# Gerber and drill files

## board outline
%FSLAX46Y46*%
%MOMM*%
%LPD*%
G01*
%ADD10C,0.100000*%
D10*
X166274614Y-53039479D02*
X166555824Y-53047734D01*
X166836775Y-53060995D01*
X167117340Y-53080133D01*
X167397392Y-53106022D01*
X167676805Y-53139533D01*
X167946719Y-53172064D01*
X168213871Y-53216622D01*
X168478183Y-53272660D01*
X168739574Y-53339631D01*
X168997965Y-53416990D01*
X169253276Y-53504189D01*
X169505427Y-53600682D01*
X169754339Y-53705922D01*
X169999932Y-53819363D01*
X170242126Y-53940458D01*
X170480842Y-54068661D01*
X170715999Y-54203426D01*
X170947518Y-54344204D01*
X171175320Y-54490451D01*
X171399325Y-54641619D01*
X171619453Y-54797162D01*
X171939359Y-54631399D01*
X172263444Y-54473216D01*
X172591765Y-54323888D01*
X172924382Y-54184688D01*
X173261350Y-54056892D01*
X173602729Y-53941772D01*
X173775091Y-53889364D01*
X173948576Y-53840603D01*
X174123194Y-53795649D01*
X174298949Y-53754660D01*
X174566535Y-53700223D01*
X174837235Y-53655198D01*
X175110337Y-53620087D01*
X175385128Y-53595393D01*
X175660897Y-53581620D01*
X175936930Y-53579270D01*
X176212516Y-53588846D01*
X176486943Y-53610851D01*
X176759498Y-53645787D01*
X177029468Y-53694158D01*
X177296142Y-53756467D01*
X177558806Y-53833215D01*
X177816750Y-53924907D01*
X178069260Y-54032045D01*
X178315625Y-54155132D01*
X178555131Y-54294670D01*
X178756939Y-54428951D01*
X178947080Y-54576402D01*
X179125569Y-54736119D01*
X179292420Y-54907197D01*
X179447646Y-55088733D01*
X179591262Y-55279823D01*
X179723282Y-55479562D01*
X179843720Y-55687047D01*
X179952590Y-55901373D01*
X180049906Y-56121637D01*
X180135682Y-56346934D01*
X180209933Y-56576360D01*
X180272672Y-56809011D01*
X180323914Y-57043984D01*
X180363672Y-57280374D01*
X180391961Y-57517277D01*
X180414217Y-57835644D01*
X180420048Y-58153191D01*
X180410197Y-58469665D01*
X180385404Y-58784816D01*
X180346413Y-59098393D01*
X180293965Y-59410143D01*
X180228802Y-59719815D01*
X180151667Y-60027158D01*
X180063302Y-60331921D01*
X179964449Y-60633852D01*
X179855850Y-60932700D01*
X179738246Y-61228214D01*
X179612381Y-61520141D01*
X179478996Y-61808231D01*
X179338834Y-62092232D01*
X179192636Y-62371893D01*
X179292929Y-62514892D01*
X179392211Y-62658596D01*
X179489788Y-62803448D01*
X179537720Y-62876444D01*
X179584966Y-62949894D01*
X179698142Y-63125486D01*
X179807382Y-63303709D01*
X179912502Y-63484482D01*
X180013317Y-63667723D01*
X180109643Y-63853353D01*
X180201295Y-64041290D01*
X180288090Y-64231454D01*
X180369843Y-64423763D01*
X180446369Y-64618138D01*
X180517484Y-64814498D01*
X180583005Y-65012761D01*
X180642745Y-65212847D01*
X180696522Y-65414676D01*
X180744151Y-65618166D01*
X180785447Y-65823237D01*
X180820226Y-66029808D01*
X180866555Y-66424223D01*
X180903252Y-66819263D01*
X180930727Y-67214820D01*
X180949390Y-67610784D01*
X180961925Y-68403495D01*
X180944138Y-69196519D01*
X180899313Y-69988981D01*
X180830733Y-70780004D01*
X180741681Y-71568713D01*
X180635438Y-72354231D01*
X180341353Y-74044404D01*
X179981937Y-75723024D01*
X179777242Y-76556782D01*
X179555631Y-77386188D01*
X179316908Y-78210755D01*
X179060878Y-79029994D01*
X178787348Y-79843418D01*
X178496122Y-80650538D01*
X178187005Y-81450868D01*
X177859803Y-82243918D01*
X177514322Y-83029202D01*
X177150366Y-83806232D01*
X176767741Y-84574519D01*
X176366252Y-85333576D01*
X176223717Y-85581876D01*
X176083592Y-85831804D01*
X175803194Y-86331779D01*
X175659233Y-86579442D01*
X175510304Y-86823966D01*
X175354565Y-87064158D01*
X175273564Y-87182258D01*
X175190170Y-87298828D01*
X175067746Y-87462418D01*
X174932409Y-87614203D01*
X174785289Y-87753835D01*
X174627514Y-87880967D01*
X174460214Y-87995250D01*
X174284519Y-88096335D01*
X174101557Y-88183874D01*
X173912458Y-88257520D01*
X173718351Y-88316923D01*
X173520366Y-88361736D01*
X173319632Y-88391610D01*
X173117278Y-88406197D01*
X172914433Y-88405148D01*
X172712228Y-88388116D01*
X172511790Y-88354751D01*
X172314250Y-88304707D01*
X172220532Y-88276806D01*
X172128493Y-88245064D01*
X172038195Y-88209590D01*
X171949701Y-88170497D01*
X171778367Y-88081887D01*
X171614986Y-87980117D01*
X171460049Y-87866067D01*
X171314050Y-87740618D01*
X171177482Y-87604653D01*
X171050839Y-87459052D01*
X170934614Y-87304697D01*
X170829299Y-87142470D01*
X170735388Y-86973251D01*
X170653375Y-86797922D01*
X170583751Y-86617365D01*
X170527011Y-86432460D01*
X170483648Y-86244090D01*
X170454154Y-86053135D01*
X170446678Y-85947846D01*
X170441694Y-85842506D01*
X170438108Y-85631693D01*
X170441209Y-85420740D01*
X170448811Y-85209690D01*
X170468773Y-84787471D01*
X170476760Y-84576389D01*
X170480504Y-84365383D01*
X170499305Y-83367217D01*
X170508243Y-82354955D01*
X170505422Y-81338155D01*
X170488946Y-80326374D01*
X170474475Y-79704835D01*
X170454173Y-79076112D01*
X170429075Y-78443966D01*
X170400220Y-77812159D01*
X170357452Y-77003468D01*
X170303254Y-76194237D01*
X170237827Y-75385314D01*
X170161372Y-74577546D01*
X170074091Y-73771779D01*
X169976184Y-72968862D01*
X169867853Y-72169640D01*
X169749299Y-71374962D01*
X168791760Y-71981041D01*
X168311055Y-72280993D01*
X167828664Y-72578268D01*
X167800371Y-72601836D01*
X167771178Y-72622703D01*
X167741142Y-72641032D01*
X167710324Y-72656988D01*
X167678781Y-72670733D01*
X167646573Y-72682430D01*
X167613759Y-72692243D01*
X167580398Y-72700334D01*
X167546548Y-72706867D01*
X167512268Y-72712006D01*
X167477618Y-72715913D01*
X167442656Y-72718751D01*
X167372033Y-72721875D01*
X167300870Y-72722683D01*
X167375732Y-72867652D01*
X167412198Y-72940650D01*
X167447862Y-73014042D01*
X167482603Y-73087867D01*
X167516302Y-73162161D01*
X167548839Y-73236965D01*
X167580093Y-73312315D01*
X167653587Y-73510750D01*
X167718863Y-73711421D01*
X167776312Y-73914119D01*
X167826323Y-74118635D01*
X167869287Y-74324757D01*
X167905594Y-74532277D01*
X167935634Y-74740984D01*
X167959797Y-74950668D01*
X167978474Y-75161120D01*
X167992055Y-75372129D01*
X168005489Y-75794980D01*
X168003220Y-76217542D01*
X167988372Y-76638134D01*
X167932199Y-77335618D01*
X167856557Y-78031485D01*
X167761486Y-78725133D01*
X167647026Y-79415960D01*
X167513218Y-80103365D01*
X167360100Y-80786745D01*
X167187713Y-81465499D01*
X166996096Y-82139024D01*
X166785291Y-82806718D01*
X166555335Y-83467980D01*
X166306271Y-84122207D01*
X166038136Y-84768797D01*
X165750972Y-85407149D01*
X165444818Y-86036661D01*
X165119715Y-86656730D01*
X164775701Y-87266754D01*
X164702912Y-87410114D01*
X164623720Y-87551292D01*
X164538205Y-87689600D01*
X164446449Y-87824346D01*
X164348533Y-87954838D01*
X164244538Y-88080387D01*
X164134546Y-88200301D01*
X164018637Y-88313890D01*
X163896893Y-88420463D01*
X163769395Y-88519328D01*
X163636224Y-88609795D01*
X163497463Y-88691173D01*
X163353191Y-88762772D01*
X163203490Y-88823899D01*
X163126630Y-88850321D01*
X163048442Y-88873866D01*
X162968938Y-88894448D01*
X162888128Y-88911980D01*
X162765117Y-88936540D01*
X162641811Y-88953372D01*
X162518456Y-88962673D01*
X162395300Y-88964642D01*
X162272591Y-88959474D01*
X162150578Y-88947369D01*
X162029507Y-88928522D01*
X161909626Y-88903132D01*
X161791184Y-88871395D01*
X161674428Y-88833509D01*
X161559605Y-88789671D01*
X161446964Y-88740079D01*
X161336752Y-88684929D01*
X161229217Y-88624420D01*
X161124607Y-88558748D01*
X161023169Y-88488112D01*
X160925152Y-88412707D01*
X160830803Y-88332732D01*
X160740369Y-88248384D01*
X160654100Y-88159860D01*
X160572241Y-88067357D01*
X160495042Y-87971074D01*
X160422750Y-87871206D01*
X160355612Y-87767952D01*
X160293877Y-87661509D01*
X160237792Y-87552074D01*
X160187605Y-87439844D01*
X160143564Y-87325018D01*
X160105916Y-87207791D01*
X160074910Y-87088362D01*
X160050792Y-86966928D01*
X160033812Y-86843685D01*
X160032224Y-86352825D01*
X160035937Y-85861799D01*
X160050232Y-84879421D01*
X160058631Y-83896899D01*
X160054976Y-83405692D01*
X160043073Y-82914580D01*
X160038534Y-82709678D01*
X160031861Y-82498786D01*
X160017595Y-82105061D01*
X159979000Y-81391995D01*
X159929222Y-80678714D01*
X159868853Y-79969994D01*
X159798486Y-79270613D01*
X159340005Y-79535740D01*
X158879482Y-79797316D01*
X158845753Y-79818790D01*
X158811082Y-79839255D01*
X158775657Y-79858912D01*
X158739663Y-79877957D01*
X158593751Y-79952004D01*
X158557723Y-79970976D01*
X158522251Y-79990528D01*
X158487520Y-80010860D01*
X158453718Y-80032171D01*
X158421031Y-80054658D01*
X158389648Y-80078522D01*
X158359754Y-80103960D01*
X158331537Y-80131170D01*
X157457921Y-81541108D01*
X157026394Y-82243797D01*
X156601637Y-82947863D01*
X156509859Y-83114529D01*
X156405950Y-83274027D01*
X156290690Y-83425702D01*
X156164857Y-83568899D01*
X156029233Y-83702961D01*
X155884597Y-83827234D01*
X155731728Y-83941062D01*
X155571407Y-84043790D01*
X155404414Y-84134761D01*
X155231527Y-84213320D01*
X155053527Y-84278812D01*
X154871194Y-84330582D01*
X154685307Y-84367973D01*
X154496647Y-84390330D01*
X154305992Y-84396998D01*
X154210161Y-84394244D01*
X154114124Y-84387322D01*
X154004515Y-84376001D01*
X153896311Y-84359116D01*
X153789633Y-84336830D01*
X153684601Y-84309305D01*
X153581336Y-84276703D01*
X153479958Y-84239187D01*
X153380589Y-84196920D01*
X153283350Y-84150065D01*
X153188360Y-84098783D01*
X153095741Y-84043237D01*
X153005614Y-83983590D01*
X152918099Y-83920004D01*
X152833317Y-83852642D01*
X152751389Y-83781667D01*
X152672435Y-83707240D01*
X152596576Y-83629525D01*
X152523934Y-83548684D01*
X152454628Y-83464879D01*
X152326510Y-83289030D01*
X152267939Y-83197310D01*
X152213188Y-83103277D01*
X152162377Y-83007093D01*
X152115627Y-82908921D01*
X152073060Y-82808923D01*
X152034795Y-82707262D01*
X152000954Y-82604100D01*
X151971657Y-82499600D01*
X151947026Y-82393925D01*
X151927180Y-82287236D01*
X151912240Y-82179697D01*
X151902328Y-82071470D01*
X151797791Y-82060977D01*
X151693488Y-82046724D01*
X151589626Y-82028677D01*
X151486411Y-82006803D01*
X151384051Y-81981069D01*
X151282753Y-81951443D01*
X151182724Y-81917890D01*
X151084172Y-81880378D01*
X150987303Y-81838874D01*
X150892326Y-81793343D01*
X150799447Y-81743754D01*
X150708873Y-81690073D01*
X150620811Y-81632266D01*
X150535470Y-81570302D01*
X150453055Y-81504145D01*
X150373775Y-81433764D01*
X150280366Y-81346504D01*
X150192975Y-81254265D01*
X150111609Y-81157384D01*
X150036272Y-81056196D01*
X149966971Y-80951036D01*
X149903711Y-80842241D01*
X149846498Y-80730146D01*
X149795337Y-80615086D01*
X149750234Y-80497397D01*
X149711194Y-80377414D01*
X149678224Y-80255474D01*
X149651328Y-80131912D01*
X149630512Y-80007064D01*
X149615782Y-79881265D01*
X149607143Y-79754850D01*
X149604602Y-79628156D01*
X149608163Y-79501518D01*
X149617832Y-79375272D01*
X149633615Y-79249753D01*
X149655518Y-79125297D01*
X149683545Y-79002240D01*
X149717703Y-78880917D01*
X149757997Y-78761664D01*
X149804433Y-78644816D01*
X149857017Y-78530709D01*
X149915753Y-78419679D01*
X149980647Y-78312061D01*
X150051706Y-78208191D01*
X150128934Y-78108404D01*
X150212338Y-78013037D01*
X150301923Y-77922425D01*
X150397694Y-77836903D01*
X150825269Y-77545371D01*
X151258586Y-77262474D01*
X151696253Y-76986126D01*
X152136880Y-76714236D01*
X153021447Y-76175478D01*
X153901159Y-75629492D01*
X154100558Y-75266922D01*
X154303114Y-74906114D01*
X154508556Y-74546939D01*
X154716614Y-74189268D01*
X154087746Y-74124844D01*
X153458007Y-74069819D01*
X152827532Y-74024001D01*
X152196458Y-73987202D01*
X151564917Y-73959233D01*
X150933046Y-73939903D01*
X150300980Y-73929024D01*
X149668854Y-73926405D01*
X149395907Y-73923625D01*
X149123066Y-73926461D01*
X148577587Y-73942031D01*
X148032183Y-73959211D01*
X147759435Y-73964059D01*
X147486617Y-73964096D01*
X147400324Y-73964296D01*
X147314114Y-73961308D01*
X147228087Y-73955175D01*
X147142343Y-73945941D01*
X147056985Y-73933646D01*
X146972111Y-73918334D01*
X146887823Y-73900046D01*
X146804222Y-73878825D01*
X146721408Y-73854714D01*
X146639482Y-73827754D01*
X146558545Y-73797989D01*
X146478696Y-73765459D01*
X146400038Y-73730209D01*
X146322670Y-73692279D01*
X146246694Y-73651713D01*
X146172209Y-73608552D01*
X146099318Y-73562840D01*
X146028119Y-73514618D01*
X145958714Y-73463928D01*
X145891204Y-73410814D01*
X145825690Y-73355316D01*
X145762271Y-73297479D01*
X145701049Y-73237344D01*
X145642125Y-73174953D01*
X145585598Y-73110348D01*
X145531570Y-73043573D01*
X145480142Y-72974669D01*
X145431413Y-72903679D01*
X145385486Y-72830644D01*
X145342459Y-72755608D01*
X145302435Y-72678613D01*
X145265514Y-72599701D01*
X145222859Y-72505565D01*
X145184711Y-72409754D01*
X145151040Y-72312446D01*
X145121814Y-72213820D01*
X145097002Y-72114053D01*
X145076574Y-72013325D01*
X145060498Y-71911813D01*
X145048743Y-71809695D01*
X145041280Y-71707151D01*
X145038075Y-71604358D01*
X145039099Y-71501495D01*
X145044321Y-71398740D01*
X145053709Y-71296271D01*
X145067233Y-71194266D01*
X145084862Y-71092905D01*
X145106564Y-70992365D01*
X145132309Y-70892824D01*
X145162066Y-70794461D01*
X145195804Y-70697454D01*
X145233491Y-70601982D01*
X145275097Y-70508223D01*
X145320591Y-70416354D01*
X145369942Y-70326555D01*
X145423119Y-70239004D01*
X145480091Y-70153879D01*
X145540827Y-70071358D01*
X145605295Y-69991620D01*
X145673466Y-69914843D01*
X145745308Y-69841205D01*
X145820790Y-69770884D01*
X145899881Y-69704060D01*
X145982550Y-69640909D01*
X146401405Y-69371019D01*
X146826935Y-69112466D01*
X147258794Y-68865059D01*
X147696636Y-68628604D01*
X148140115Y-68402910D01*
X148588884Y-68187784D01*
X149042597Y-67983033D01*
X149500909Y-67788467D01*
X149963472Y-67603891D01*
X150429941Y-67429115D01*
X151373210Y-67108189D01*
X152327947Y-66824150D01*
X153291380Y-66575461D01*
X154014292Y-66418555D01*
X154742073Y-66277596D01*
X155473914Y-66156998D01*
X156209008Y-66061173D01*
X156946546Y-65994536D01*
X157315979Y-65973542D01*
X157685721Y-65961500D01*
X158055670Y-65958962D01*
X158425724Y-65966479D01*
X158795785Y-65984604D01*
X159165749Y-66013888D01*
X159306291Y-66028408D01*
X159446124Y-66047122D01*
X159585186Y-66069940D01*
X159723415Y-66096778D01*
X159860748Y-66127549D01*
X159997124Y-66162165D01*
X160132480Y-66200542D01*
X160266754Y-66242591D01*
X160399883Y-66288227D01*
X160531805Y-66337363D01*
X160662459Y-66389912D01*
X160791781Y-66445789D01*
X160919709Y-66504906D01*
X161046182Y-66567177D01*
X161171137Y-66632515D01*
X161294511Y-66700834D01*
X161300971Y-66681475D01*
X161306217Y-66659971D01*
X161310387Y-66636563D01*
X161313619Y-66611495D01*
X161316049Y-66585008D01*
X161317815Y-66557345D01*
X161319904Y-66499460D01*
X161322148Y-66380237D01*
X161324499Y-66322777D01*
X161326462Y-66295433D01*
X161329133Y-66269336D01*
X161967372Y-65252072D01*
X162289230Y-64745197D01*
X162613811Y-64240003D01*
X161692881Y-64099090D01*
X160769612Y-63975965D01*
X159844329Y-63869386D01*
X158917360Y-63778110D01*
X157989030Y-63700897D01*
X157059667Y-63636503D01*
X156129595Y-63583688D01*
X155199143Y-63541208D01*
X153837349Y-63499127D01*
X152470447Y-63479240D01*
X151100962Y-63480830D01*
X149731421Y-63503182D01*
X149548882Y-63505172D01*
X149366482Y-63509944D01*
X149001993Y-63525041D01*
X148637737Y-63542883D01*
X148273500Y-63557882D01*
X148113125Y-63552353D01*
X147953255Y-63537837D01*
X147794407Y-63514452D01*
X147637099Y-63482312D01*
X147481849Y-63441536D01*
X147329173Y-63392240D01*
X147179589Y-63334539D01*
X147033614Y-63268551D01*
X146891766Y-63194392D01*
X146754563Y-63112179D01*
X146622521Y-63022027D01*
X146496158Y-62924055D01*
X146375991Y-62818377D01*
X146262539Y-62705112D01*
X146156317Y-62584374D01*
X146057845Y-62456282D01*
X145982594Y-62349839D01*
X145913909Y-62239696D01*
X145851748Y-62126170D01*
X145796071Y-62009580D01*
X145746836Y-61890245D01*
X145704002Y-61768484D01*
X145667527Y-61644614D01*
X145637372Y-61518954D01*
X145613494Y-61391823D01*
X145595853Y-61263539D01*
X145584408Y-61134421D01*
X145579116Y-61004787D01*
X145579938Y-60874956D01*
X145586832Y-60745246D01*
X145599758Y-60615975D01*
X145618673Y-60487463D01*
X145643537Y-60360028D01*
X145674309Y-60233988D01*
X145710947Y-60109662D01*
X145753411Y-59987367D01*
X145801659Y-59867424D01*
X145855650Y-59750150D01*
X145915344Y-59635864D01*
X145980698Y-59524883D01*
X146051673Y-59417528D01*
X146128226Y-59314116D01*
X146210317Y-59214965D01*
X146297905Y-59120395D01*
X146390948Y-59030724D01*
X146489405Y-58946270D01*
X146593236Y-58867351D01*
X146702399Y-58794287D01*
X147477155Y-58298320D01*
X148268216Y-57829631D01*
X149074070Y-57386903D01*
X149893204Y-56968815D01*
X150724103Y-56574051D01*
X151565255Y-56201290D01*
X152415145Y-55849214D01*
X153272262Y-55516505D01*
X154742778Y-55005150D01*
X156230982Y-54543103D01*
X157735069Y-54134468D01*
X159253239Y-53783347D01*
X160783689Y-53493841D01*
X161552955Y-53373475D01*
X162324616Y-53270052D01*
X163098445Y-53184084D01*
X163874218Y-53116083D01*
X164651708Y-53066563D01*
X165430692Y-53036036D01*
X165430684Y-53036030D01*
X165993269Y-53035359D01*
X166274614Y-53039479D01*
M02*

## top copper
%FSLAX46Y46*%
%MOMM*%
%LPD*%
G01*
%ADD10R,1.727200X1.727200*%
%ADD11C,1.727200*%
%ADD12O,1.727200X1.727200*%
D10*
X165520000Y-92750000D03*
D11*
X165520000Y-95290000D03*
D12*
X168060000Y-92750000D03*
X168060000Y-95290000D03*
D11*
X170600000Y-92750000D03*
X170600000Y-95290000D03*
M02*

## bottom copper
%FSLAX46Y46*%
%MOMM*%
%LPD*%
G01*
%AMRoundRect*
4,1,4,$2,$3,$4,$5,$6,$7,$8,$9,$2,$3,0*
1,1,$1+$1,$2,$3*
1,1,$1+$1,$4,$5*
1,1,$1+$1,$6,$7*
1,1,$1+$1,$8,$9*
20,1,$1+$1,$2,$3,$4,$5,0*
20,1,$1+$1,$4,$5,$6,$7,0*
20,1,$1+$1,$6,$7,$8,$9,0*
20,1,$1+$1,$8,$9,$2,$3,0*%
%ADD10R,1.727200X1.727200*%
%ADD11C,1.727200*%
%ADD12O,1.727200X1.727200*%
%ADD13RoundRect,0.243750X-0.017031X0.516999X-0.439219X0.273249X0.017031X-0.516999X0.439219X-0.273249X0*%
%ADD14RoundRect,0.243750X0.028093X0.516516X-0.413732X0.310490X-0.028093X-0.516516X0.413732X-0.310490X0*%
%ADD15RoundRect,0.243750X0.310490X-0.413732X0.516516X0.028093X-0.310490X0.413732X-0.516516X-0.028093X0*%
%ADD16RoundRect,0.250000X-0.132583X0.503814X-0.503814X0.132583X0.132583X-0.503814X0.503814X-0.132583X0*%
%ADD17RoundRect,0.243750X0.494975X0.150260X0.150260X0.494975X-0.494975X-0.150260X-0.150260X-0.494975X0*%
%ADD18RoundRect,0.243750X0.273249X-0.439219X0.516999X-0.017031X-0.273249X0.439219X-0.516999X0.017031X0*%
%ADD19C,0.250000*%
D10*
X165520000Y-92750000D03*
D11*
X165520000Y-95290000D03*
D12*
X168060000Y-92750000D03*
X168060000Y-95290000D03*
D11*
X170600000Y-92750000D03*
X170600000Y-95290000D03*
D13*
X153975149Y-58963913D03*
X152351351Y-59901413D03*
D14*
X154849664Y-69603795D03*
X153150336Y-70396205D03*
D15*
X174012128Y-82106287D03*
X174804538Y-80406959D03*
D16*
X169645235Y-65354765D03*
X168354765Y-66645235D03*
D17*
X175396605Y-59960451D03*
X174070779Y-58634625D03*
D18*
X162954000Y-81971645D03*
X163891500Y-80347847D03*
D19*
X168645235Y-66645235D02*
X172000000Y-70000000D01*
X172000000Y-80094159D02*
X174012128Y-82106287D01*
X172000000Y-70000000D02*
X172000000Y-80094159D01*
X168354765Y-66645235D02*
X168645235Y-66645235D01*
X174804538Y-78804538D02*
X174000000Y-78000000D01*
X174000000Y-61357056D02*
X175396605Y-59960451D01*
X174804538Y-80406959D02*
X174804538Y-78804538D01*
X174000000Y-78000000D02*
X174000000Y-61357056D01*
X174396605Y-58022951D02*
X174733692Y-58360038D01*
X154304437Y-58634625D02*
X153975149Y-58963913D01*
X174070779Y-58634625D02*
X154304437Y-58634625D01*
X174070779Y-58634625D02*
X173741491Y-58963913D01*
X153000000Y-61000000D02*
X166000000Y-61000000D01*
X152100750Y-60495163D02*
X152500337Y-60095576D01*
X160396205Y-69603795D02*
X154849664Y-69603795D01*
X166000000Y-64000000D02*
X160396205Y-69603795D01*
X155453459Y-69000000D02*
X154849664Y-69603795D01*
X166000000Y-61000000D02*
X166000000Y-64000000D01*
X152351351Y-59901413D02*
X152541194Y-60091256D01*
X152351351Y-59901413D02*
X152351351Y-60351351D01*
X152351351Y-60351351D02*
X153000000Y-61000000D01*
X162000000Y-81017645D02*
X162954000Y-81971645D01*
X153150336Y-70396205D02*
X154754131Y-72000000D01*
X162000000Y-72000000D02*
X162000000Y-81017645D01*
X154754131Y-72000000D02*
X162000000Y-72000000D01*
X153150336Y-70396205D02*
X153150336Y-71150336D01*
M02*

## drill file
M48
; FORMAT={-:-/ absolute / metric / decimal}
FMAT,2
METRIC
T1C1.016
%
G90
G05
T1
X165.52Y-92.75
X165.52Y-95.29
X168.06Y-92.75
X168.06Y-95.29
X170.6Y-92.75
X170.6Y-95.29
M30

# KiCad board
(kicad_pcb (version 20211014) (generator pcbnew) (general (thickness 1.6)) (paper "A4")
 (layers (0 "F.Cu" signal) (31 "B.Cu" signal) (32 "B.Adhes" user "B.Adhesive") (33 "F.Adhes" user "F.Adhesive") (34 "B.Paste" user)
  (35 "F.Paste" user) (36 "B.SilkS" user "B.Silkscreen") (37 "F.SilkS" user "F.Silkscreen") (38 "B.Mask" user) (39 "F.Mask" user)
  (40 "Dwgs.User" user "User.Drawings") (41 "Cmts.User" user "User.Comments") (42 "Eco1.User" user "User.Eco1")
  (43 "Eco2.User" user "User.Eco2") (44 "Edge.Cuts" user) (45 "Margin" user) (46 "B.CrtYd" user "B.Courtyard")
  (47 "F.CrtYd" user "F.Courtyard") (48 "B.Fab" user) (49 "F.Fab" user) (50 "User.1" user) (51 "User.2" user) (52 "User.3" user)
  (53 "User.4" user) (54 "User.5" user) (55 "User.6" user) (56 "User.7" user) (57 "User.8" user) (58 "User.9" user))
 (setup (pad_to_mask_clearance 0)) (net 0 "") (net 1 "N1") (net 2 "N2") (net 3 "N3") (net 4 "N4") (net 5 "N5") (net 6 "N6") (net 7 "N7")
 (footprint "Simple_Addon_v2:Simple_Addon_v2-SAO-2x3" (layer "F.Cu") (at 168 94)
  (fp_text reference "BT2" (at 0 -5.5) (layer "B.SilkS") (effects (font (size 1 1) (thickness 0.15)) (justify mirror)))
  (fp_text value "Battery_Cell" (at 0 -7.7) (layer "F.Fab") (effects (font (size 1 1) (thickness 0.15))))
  (pad "1" thru_hole rect locked (at -2.48 -1.25 270) (size 1.7272 1.7272) (drill 1.016) (layers *.Cu *.Mask) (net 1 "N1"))
  (pad "2" thru_hole circle locked (at -2.48 1.29 270) (size 1.7272 1.7272) (drill 1.016) (layers *.Cu *.Mask) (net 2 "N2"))
  (pad "3" thru_hole oval locked (at 0.06 -1.25 270) (size 1.7272 1.7272) (drill 1.016) (layers *.Cu *.Mask))
  (pad "4" thru_hole oval locked (at 0.06 1.29 270) (size 1.7272 1.7272) (drill 1.016) (layers *.Cu *.Mask))
  (pad "5" thru_hole circle locked (at 2.6 -1.25 270) (size 1.7272 1.7272) (drill 1.016) (layers *.Cu *.Mask))
  (pad "6" thru_hole circle locked (at 2.6 1.29 270) (size 1.7272 1.7272) (drill 1.016) (layers *.Cu *.Mask)))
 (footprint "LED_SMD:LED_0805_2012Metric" (layer "B.Cu") (at 153.16325 59.432663 -150)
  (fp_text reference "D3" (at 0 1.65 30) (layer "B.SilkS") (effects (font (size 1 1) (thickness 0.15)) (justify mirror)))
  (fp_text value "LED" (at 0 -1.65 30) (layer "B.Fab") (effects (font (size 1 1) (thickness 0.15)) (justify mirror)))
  (pad "1" smd roundrect (at -0.9375 0 210) (size 0.975 1.4) (layers "B.Cu" "B.Paste" "B.Mask") (roundrect_rratio 0.25) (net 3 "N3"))
  (pad "2" smd roundrect (at 0.9375 0 210) (size 0.975 1.4) (layers "B.Cu" "B.Paste" "B.Mask") (roundrect_rratio 0.25) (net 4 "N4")))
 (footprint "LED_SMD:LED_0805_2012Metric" (layer "B.Cu") (at 154 70 -155)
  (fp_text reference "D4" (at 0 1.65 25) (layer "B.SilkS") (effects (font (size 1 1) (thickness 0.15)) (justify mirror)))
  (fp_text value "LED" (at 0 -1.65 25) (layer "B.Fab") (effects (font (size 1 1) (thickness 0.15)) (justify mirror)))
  (pad "1" smd roundrect (at -0.9375 0 205) (size 0.975 1.4) (layers "B.Cu" "B.Paste" "B.Mask") (roundrect_rratio 0.25) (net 4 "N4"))
  (pad "2" smd roundrect (at 0.9375 0 205) (size 0.975 1.4) (layers "B.Cu" "B.Paste" "B.Mask") (roundrect_rratio 0.25) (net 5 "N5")))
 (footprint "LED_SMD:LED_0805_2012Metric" (layer "B.Cu") (at 174.408333 81.256623 65)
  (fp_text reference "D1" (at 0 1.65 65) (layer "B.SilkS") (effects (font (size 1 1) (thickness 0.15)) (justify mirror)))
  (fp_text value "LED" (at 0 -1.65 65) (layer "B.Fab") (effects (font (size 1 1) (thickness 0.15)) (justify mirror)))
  (pad "1" smd roundrect (at -0.9375 0 65) (size 0.975 1.4) (layers "B.Cu" "B.Paste" "B.Mask") (roundrect_rratio 0.25) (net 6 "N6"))
  (pad "2" smd roundrect (at 0.9375 0 65) (size 0.975 1.4) (layers "B.Cu" "B.Paste" "B.Mask") (roundrect_rratio 0.25) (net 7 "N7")))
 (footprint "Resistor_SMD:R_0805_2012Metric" (layer "B.Cu") (at 169 66 -135)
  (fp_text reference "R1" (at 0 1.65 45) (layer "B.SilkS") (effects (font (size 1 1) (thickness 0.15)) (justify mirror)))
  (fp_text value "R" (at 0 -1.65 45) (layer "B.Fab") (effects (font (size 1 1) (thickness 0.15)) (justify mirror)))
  (pad "1" smd roundrect (at -0.9125 0 225) (size 1.025 1.4) (layers "B.Cu" "B.Paste" "B.Mask") (roundrect_rratio 0.243902) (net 2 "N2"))
  (pad "2" smd roundrect (at 0.9125 0 225) (size 1.025 1.4) (layers "B.Cu" "B.Paste" "B.Mask") (roundrect_rratio 0.243902) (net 6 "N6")))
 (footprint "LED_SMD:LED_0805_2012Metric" (layer "B.Cu") (at 174.733692 59.297538 135)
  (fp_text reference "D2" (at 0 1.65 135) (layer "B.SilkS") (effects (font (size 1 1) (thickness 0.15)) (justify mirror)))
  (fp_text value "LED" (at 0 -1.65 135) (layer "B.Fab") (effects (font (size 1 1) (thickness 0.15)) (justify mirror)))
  (pad "1" smd roundrect (at -0.9375 0 135) (size 0.975 1.4) (layers "B.Cu" "B.Paste" "B.Mask") (roundrect_rratio 0.25) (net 7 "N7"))
  (pad "2" smd roundrect (at 0.9375 0 135) (size 0.975 1.4) (layers "B.Cu" "B.Paste" "B.Mask") (roundrect_rratio 0.25) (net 3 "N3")))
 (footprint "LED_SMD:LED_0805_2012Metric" (layer "B.Cu") (at 163.42275 81.159746 60)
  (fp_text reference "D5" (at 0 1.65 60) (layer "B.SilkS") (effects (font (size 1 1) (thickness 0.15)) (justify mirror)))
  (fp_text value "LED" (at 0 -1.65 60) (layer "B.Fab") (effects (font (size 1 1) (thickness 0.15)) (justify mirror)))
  (pad "1" smd roundrect (at -0.9375 0 60) (size 0.975 1.4) (layers "B.Cu" "B.Paste" "B.Mask") (roundrect_rratio 0.25) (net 5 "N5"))
  (pad "2" smd roundrect (at 0.9375 0 60) (size 0.975 1.4) (layers "B.Cu" "B.Paste" "B.Mask") (roundrect_rratio 0.25) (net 1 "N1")))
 (gr_poly
  (pts (xy 166.274614 53.039479) (xy 166.555824 53.047734) (xy 166.836775 53.060995) (xy 167.11734 53.080133) (xy 167.397392 53.106022)
   (xy 167.676805 53.139533) (xy 167.946719 53.172064) (xy 168.213871 53.216622) (xy 168.478183 53.27266) (xy 168.739574 53.339631)
   (xy 168.997965 53.41699) (xy 169.253276 53.504189) (xy 169.505427 53.600682) (xy 169.754339 53.705922) (xy 169.999932 53.819363)
   (xy 170.242126 53.940458) (xy 170.480842 54.068661) (xy 170.715999 54.203426) (xy 170.947518 54.344204) (xy 171.17532 54.490451)
   (xy 171.399325 54.641619) (xy 171.619453 54.797162) (xy 171.939359 54.631399) (xy 172.263444 54.473216) (xy 172.591765 54.323888)
   (xy 172.924382 54.184688) (xy 173.26135 54.056892) (xy 173.602729 53.941772) (xy 173.775091 53.889364) (xy 173.948576 53.840603)
   (xy 174.123194 53.795649) (xy 174.298949 53.75466) (xy 174.566535 53.700223) (xy 174.837235 53.655198) (xy 175.110337 53.620087)
   (xy 175.385128 53.595393) (xy 175.660897 53.58162) (xy 175.93693 53.57927) (xy 176.212516 53.588846) (xy 176.486943 53.610851)
   (xy 176.759498 53.645787) (xy 177.029468 53.694158) (xy 177.296142 53.756467) (xy 177.558806 53.833215) (xy 177.81675 53.924907)
   (xy 178.06926 54.032045) (xy 178.315625 54.155132) (xy 178.555131 54.29467) (xy 178.756939 54.428951) (xy 178.94708 54.576402)
   (xy 179.125569 54.736119) (xy 179.29242 54.907197) (xy 179.447646 55.088733) (xy 179.591262 55.279823) (xy 179.723282 55.479562)
   (xy 179.84372 55.687047) (xy 179.95259 55.901373) (xy 180.049906 56.121637) (xy 180.135682 56.346934) (xy 180.209933 56.57636)
   (xy 180.272672 56.809011) (xy 180.323914 57.043984) (xy 180.363672 57.280374) (xy 180.391961 57.517277) (xy 180.414217 57.835644)
   (xy 180.420048 58.153191) (xy 180.410197 58.469665) (xy 180.385404 58.784816) (xy 180.346413 59.098393) (xy 180.293965 59.410143)
   (xy 180.228802 59.719815) (xy 180.151667 60.027158) (xy 180.063302 60.331921) (xy 179.964449 60.633852) (xy 179.85585 60.9327)
   (xy 179.738246 61.228214) (xy 179.612381 61.520141) (xy 179.478996 61.808231) (xy 179.338834 62.092232) (xy 179.192636 62.371893)
   (xy 179.292929 62.514892) (xy 179.392211 62.658596) (xy 179.489788 62.803448) (xy 179.53772 62.876444) (xy 179.584966 62.949894)
   (xy 179.698142 63.125486) (xy 179.807382 63.303709) (xy 179.912502 63.484482) (xy 180.013317 63.667723) (xy 180.109643 63.853353)
   (xy 180.201295 64.04129) (xy 180.28809 64.231454) (xy 180.369843 64.423763) (xy 180.446369 64.618138) (xy 180.517484 64.814498)
   (xy 180.583005 65.012761) (xy 180.642745 65.212847) (xy 180.696522 65.414676) (xy 180.744151 65.618166) (xy 180.785447 65.823237)
   (xy 180.820226 66.029808) (xy 180.866555 66.424223) (xy 180.903252 66.819263) (xy 180.930727 67.21482) (xy 180.94939 67.610784)
   (xy 180.961925 68.403495) (xy 180.944138 69.196519) (xy 180.899313 69.988981) (xy 180.830733 70.780004) (xy 180.741681 71.568713)
   (xy 180.635438 72.354231) (xy 180.341353 74.044404) (xy 179.981937 75.723024) (xy 179.777242 76.556782) (xy 179.555631 77.386188)
   (xy 179.316908 78.210755) (xy 179.060878 79.029994) (xy 178.787348 79.843418) (xy 178.496122 80.650538) (xy 178.187005 81.450868)
   (xy 177.859803 82.243918) (xy 177.514322 83.029202) (xy 177.150366 83.806232) (xy 176.767741 84.574519) (xy 176.366252 85.333576)
   (xy 176.223717 85.581876) (xy 176.083592 85.831804) (xy 175.803194 86.331779) (xy 175.659233 86.579442) (xy 175.510304 86.823966)
   (xy 175.354565 87.064158) (xy 175.273564 87.182258) (xy 175.19017 87.298828) (xy 175.067746 87.462418) (xy 174.932409 87.614203)
   (xy 174.785289 87.753835) (xy 174.627514 87.880967) (xy 174.460214 87.99525) (xy 174.284519 88.096335) (xy 174.101557 88.183874)
   (xy 173.912458 88.25752) (xy 173.718351 88.316923) (xy 173.520366 88.361736) (xy 173.319632 88.39161) (xy 173.117278 88.406197)
   (xy 172.914433 88.405148) (xy 172.712228 88.388116) (xy 172.51179 88.354751) (xy 172.31425 88.304707) (xy 172.220532 88.276806)
   (xy 172.128493 88.245064) (xy 172.038195 88.20959) (xy 171.949701 88.170497) (xy 171.778367 88.081887) (xy 171.614986 87.980117)
   (xy 171.460049 87.866067) (xy 171.31405 87.740618) (xy 171.177482 87.604653) (xy 171.050839 87.459052) (xy 170.934614 87.304697)
   (xy 170.829299 87.14247) (xy 170.735388 86.973251) (xy 170.653375 86.797922) (xy 170.583751 86.617365) (xy 170.527011 86.43246)
   (xy 170.483648 86.24409) (xy 170.454154 86.053135) (xy 170.446678 85.947846) (xy 170.441694 85.842506) (xy 170.438108 85.631693)
   (xy 170.441209 85.42074) (xy 170.448811 85.20969) (xy 170.468773 84.787471) (xy 170.47676 84.576389) (xy 170.480504 84.365383)
   (xy 170.499305 83.367217) (xy 170.508243 82.354955) (xy 170.505422 81.338155) (xy 170.488946 80.326374) (xy 170.474475 79.704835)
   (xy 170.454173 79.076112) (xy 170.429075 78.443966) (xy 170.40022 77.812159) (xy 170.357452 77.003468) (xy 170.303254 76.194237)
   (xy 170.237827 75.385314) (xy 170.161372 74.577546) (xy 170.074091 73.771779) (xy 169.976184 72.968862) (xy 169.867853 72.16964)
   (xy 169.749299 71.374962) (xy 168.79176 71.981041) (xy 168.311055 72.280993) (xy 167.828664 72.578268) (xy 167.800371 72.601836)
   (xy 167.771178 72.622703) (xy 167.741142 72.641032) (xy 167.710324 72.656988) (xy 167.678781 72.670733) (xy 167.646573 72.68243)
   (xy 167.613759 72.692243) (xy 167.580398 72.700334) (xy 167.546548 72.706867) (xy 167.512268 72.712006) (xy 167.477618 72.715913)
   (xy 167.442656 72.718751) (xy 167.372033 72.721875) (xy 167.30087 72.722683) (xy 167.375732 72.867652) (xy 167.412198 72.94065)
   (xy 167.447862 73.014042) (xy 167.482603 73.087867) (xy 167.516302 73.162161) (xy 167.548839 73.236965) (xy 167.580093 73.312315)
   (xy 167.653587 73.51075) (xy 167.718863 73.711421) (xy 167.776312 73.914119) (xy 167.826323 74.118635) (xy 167.869287 74.324757)
   (xy 167.905594 74.532277) (xy 167.935634 74.740984) (xy 167.959797 74.950668) (xy 167.978474 75.16112) (xy 167.992055 75.372129)
   (xy 168.005489 75.79498) (xy 168.00322 76.217542) (xy 167.988372 76.638134) (xy 167.932199 77.335618) (xy 167.856557 78.031485)
   (xy 167.761486 78.725133) (xy 167.647026 79.41596) (xy 167.513218 80.103365) (xy 167.3601 80.786745) (xy 167.187713 81.465499)
   (xy 166.996096 82.139024) (xy 166.785291 82.806718) (xy 166.555335 83.46798) (xy 166.306271 84.122207) (xy 166.038136 84.768797)
   (xy 165.750972 85.407149) (xy 165.444818 86.036661) (xy 165.119715 86.65673) (xy 164.775701 87.266754) (xy 164.702912 87.410114)
   (xy 164.62372 87.551292) (xy 164.538205 87.6896) (xy 164.446449 87.824346) (xy 164.348533 87.954838) (xy 164.244538 88.080387)
   (xy 164.134546 88.200301) (xy 164.018637 88.31389) (xy 163.896893 88.420463) (xy 163.769395 88.519328) (xy 163.636224 88.609795)
   (xy 163.497463 88.691173) (xy 163.353191 88.762772) (xy 163.20349 88.823899) (xy 163.12663 88.850321) (xy 163.048442 88.873866)
   (xy 162.968938 88.894448) (xy 162.888128 88.91198) (xy 162.765117 88.93654) (xy 162.641811 88.953372) (xy 162.518456 88.962673)
   (xy 162.3953 88.964642) (xy 162.272591 88.959474) (xy 162.150578 88.947369) (xy 162.029507 88.928522) (xy 161.909626 88.903132)
   (xy 161.791184 88.871395) (xy 161.674428 88.833509) (xy 161.559605 88.789671) (xy 161.446964 88.740079) (xy 161.336752 88.684929)
   (xy 161.229217 88.62442) (xy 161.124607 88.558748) (xy 161.023169 88.488112) (xy 160.925152 88.412707) (xy 160.830803 88.332732)
   (xy 160.740369 88.248384) (xy 160.6541 88.15986) (xy 160.572241 88.067357) (xy 160.495042 87.971074) (xy 160.42275 87.871206)
   (xy 160.355612 87.767952) (xy 160.293877 87.661509) (xy 160.237792 87.552074) (xy 160.187605 87.439844) (xy 160.143564 87.325018)
   (xy 160.105916 87.207791) (xy 160.07491 87.088362) (xy 160.050792 86.966928) (xy 160.033812 86.843685) (xy 160.032224 86.352825)
   (xy 160.035937 85.861799) (xy 160.050232 84.879421) (xy 160.058631 83.896899) (xy 160.054976 83.405692) (xy 160.043073 82.91458)
   (xy 160.038534 82.709678) (xy 160.031861 82.498786) (xy 160.017595 82.105061) (xy 159.979 81.391995) (xy 159.929222 80.678714)
   (xy 159.868853 79.969994) (xy 159.798486 79.270613) (xy 159.340005 79.53574) (xy 158.879482 79.797316) (xy 158.845753 79.81879)
   (xy 158.811082 79.839255) (xy 158.775657 79.858912) (xy 158.739663 79.877957) (xy 158.593751 79.952004) (xy 158.557723 79.970976)
   (xy 158.522251 79.990528) (xy 158.48752 80.01086) (xy 158.453718 80.032171) (xy 158.421031 80.054658) (xy 158.389648 80.078522)
   (xy 158.359754 80.10396) (xy 158.331537 80.13117) (xy 157.457921 81.541108) (xy 157.026394 82.243797) (xy 156.601637 82.947863)
   (xy 156.509859 83.114529) (xy 156.40595 83.274027) (xy 156.29069 83.425702) (xy 156.164857 83.568899) (xy 156.029233 83.702961)
   (xy 155.884597 83.827234) (xy 155.731728 83.941062) (xy 155.571407 84.04379) (xy 155.404414 84.134761) (xy 155.231527 84.21332)
   (xy 155.053527 84.278812) (xy 154.871194 84.330582) (xy 154.685307 84.367973) (xy 154.496647 84.39033) (xy 154.305992 84.396998)
   (xy 154.210161 84.394244) (xy 154.114124 84.387322) (xy 154.004515 84.376001) (xy 153.896311 84.359116) (xy 153.789633 84.33683)
   (xy 153.684601 84.309305) (xy 153.581336 84.276703) (xy 153.479958 84.239187) (xy 153.380589 84.19692) (xy 153.28335 84.150065)
   (xy 153.18836 84.098783) (xy 153.095741 84.043237) (xy 153.005614 83.98359) (xy 152.918099 83.920004) (xy 152.833317 83.852642)
   (xy 152.751389 83.781667) (xy 152.672435 83.70724) (xy 152.596576 83.629525) (xy 152.523934 83.548684) (xy 152.454628 83.464879)
   (xy 152.32651 83.28903) (xy 152.267939 83.19731) (xy 152.213188 83.103277) (xy 152.162377 83.007093) (xy 152.115627 82.908921)
   (xy 152.07306 82.808923) (xy 152.034795 82.707262) (xy 152.000954 82.6041) (xy 151.971657 82.4996) (xy 151.947026 82.393925)
   (xy 151.92718 82.287236) (xy 151.91224 82.179697) (xy 151.902328 82.07147) (xy 151.797791 82.060977) (xy 151.693488 82.046724)
   (xy 151.589626 82.028677) (xy 151.486411 82.006803) (xy 151.384051 81.981069) (xy 151.282753 81.951443) (xy 151.182724 81.91789)
   (xy 151.084172 81.880378) (xy 150.987303 81.838874) (xy 150.892326 81.793343) (xy 150.799447 81.743754) (xy 150.708873 81.690073)
   (xy 150.620811 81.632266) (xy 150.53547 81.570302) (xy 150.453055 81.504145) (xy 150.373775 81.433764) (xy 150.280366 81.346504)
   (xy 150.192975 81.254265) (xy 150.111609 81.157384) (xy 150.036272 81.056196) (xy 149.966971 80.951036) (xy 149.903711 80.842241)
   (xy 149.846498 80.730146) (xy 149.795337 80.615086) (xy 149.750234 80.497397) (xy 149.711194 80.377414) (xy 149.678224 80.255474)
   (xy 149.651328 80.131912) (xy 149.630512 80.007064) (xy 149.615782 79.881265) (xy 149.607143 79.75485) (xy 149.604602 79.628156)
   (xy 149.608163 79.501518) (xy 149.617832 79.375272) (xy 149.633615 79.249753) (xy 149.655518 79.125297) (xy 149.683545 79.00224)
   (xy 149.717703 78.880917) (xy 149.757997 78.761664) (xy 149.804433 78.644816) (xy 149.857017 78.530709) (xy 149.915753 78.419679)
   (xy 149.980647 78.312061) (xy 150.051706 78.208191) (xy 150.128934 78.108404) (xy 150.212338 78.013037) (xy 150.301923 77.922425)
   (xy 150.397694 77.836903) (xy 150.825269 77.545371) (xy 151.258586 77.262474) (xy 151.696253 76.986126) (xy 152.13688 76.714236)
   (xy 153.021447 76.175478) (xy 153.901159 75.629492) (xy 154.100558 75.266922) (xy 154.303114 74.906114) (xy 154.508556 74.546939)
   (xy 154.716614 74.189268) (xy 154.087746 74.124844) (xy 153.458007 74.069819) (xy 152.827532 74.024001) (xy 152.196458 73.987202)
   (xy 151.564917 73.959233) (xy 150.933046 73.939903) (xy 150.30098 73.929024) (xy 149.668854 73.926405) (xy 149.395907 73.923625)
   (xy 149.123066 73.926461) (xy 148.577587 73.942031) (xy 148.032183 73.959211) (xy 147.759435 73.964059) (xy 147.486617 73.964096)
   (xy 147.400324 73.964296) (xy 147.314114 73.961308) (xy 147.228087 73.955175) (xy 147.142343 73.945941) (xy 147.056985 73.933646)
   (xy 146.972111 73.918334) (xy 146.887823 73.900046) (xy 146.804222 73.878825) (xy 146.721408 73.854714) (xy 146.639482 73.827754)
   (xy 146.558545 73.797989) (xy 146.478696 73.765459) (xy 146.400038 73.730209) (xy 146.32267 73.692279) (xy 146.246694 73.651713)
   (xy 146.172209 73.608552) (xy 146.099318 73.56284) (xy 146.028119 73.514618) (xy 145.958714 73.463928) (xy 145.891204 73.410814)
   (xy 145.82569 73.355316) (xy 145.762271 73.297479) (xy 145.701049 73.237344) (xy 145.642125 73.174953) (xy 145.585598 73.110348)
   (xy 145.53157 73.043573) (xy 145.480142 72.974669) (xy 145.431413 72.903679) (xy 145.385486 72.830644) (xy 145.342459 72.755608)
   (xy 145.302435 72.678613) (xy 145.265514 72.599701) (xy 145.222859 72.505565) (xy 145.184711 72.409754) (xy 145.15104 72.312446)
   (xy 145.121814 72.21382) (xy 145.097002 72.114053) (xy 145.076574 72.013325) (xy 145.060498 71.911813) (xy 145.048743 71.809695)
   (xy 145.04128 71.707151) (xy 145.038075 71.604358) (xy 145.039099 71.501495) (xy 145.044321 71.39874) (xy 145.053709 71.296271)
   (xy 145.067233 71.194266) (xy 145.084862 71.092905) (xy 145.106564 70.992365) (xy 145.132309 70.892824) (xy 145.162066 70.794461)
   (xy 145.195804 70.697454) (xy 145.233491 70.601982) (xy 145.275097 70.508223) (xy 145.320591 70.416354) (xy 145.369942 70.326555)
   (xy 145.423119 70.239004) (xy 145.480091 70.153879) (xy 145.540827 70.071358) (xy 145.605295 69.99162) (xy 145.673466 69.914843)
   (xy 145.745308 69.841205) (xy 145.82079 69.770884) (xy 145.899881 69.70406) (xy 145.98255 69.640909) (xy 146.401405 69.371019)
   (xy 146.826935 69.112466) (xy 147.258794 68.865059) (xy 147.696636 68.628604) (xy 148.140115 68.40291) (xy 148.588884 68.187784)
   (xy 149.042597 67.983033) (xy 149.500909 67.788467) (xy 149.963472 67.603891) (xy 150.429941 67.429115) (xy 151.37321 67.108189)
   (xy 152.327947 66.82415) (xy 153.29138 66.575461) (xy 154.014292 66.418555) (xy 154.742073 66.277596) (xy 155.473914 66.156998)
   (xy 156.209008 66.061173) (xy 156.946546 65.994536) (xy 157.315979 65.973542) (xy 157.685721 65.9615) (xy 158.05567 65.958962)
   (xy 158.425724 65.966479) (xy 158.795785 65.984604) (xy 159.165749 66.013888) (xy 159.306291 66.028408) (xy 159.446124 66.047122)
   (xy 159.585186 66.06994) (xy 159.723415 66.096778) (xy 159.860748 66.127549) (xy 159.997124 66.162165) (xy 160.13248 66.200542)
   (xy 160.266754 66.242591) (xy 160.399883 66.288227) (xy 160.531805 66.337363) (xy 160.662459 66.389912) (xy 160.791781 66.445789)
   (xy 160.919709 66.504906) (xy 161.046182 66.567177) (xy 161.171137 66.632515) (xy 161.294511 66.700834) (xy 161.300971 66.681475)
   (xy 161.306217 66.659971) (xy 161.310387 66.636563) (xy 161.313619 66.611495) (xy 161.316049 66.585008) (xy 161.317815 66.557345)
   (xy 161.319904 66.49946) (xy 161.322148 66.380237) (xy 161.324499 66.322777) (xy 161.326462 66.295433) (xy 161.329133 66.269336)
   (xy 161.967372 65.252072) (xy 162.28923 64.745197) (xy 162.613811 64.240003) (xy 161.692881 64.09909) (xy 160.769612 63.975965)
   (xy 159.844329 63.869386) (xy 158.91736 63.77811) (xy 157.98903 63.700897) (xy 157.059667 63.636503) (xy 156.129595 63.583688)
   (xy 155.199143 63.541208) (xy 153.837349 63.499127) (xy 152.470447 63.47924) (xy 151.100962 63.48083) (xy 149.731421 63.503182)
   (xy 149.548882 63.505172) (xy 149.366482 63.509944) (xy 149.001993 63.525041) (xy 148.637737 63.542883) (xy 148.2735 63.557882)
   (xy 148.113125 63.552353) (xy 147.953255 63.537837) (xy 147.794407 63.514452) (xy 147.637099 63.482312) (xy 147.481849 63.441536)
   (xy 147.329173 63.39224) (xy 147.179589 63.334539) (xy 147.033614 63.268551) (xy 146.891766 63.194392) (xy 146.754563 63.112179)
   (xy 146.622521 63.022027) (xy 146.496158 62.924055) (xy 146.375991 62.818377) (xy 146.262539 62.705112) (xy 146.156317 62.584374)
   (xy 146.057845 62.456282) (xy 145.982594 62.349839) (xy 145.913909 62.239696) (xy 145.851748 62.12617) (xy 145.796071 62.00958)
   (xy 145.746836 61.890245) (xy 145.704002 61.768484) (xy 145.667527 61.644614) (xy 145.637372 61.518954) (xy 145.613494 61.391823)
   (xy 145.595853 61.263539) (xy 145.584408 61.134421) (xy 145.579116 61.004787) (xy 145.579938 60.874956) (xy 145.586832 60.745246)
   (xy 145.599758 60.615975) (xy 145.618673 60.487463) (xy 145.643537 60.360028) (xy 145.674309 60.233988) (xy 145.710947 60.109662)
   (xy 145.753411 59.987367) (xy 145.801659 59.867424) (xy 145.85565 59.75015) (xy 145.915344 59.635864) (xy 145.980698 59.524883)
   (xy 146.051673 59.417528) (xy 146.128226 59.314116) (xy 146.210317 59.214965) (xy 146.297905 59.120395) (xy 146.390948 59.030724)
   (xy 146.489405 58.94627) (xy 146.593236 58.867351) (xy 146.702399 58.794287) (xy 147.477155 58.29832) (xy 148.268216 57.829631)
   (xy 149.07407 57.386903) (xy 149.893204 56.968815) (xy 150.724103 56.574051) (xy 151.565255 56.20129) (xy 152.415145 55.849214)
   (xy 153.272262 55.516505) (xy 154.742778 55.00515) (xy 156.230982 54.543103) (xy 157.735069 54.134468) (xy 159.253239 53.783347)
   (xy 160.783689 53.493841) (xy 161.552955 53.373475) (xy 162.324616 53.270052) (xy 163.098445 53.184084) (xy 163.874218 53.116083)
   (xy 164.651708 53.066563) (xy 165.430692 53.036036) (xy 165.430684 53.03603) (xy 165.993269 53.035359))
  (layer "Edge.Cuts") (width 0) (fill none))
 (segment (start 168.645235 66.645235) (end 172 70) (width 0.25) (layer "B.Cu") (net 6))
 (segment (start 172 80.094159) (end 174.012128 82.106287) (width 0.25) (layer "B.Cu") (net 6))
 (segment (start 172 70) (end 172 80.094159) (width 0.25) (layer "B.Cu") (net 6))
 (segment (start 168.354765 66.645235) (end 168.645235 66.645235) (width 0.25) (layer "B.Cu") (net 6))
 (segment (start 174.804538 78.804538) (end 174 78) (width 0.25) (layer "B.Cu") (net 7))
 (segment (start 174 61.357056) (end 175.396605 59.960451) (width 0.25) (layer "B.Cu") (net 7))
 (segment (start 174.804538 80.406959) (end 174.804538 78.804538) (width 0.25) (layer "B.Cu") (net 7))
 (segment (start 174 78) (end 174 61.357056) (width 0.25) (layer "B.Cu") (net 7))
 (segment (start 174.396605 58.022951) (end 174.733692 58.360038) (width 0.25) (layer "B.Cu") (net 3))
 (segment (start 154.304437 58.634625) (end 153.975149 58.963913) (width 0.25) (layer "B.Cu") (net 3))
 (segment (start 174.070779 58.634625) (end 154.304437 58.634625) (width 0.25) (layer "B.Cu") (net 3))
 (segment (start 174.070779 58.634625) (end 173.741491 58.963913) (width 0.25) (layer "B.Cu") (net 3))
 (segment (start 153 61) (end 166 61) (width 0.25) (layer "B.Cu") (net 4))
 (segment (start 152.10075 60.495163) (end 152.500337 60.095576) (width 0.25) (layer "B.Cu") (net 4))
 (segment (start 160.396205 69.603795) (end 154.849664 69.603795) (width 0.25) (layer "B.Cu") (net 4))
 (segment (start 166 64) (end 160.396205 69.603795) (width 0.25) (layer "B.Cu") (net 4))
 (segment (start 155.453459 69) (end 154.849664 69.603795) (width 0.25) (layer "B.Cu") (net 4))
 (segment (start 166 61) (end 166 64) (width 0.25) (layer "B.Cu") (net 4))
 (segment (start 152.351351 59.901413) (end 152.541194 60.091256) (width 0.25) (layer "B.Cu") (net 4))
 (segment (start 152.351351 59.901413) (end 152.351351 60.351351) (width 0.25) (layer "B.Cu") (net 4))
 (segment (start 152.351351 60.351351) (end 153 61) (width 0.25) (layer "B.Cu") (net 4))
 (segment (start 162 81.017645) (end 162.954 81.971645) (width 0.25) (layer "B.Cu") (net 5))
 (segment (start 153.150336 70.396205) (end 154.754131 72) (width 0.25) (layer "B.Cu") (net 5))
 (segment (start 162 72) (end 162 81.017645) (width 0.25) (layer "B.Cu") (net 5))
 (segment (start 154.754131 72) (end 162 72) (width 0.25) (layer "B.Cu") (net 5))
 (segment (start 153.150336 70.396205) (end 153.150336 71.150336) (width 0.25) (layer "B.Cu") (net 5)))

